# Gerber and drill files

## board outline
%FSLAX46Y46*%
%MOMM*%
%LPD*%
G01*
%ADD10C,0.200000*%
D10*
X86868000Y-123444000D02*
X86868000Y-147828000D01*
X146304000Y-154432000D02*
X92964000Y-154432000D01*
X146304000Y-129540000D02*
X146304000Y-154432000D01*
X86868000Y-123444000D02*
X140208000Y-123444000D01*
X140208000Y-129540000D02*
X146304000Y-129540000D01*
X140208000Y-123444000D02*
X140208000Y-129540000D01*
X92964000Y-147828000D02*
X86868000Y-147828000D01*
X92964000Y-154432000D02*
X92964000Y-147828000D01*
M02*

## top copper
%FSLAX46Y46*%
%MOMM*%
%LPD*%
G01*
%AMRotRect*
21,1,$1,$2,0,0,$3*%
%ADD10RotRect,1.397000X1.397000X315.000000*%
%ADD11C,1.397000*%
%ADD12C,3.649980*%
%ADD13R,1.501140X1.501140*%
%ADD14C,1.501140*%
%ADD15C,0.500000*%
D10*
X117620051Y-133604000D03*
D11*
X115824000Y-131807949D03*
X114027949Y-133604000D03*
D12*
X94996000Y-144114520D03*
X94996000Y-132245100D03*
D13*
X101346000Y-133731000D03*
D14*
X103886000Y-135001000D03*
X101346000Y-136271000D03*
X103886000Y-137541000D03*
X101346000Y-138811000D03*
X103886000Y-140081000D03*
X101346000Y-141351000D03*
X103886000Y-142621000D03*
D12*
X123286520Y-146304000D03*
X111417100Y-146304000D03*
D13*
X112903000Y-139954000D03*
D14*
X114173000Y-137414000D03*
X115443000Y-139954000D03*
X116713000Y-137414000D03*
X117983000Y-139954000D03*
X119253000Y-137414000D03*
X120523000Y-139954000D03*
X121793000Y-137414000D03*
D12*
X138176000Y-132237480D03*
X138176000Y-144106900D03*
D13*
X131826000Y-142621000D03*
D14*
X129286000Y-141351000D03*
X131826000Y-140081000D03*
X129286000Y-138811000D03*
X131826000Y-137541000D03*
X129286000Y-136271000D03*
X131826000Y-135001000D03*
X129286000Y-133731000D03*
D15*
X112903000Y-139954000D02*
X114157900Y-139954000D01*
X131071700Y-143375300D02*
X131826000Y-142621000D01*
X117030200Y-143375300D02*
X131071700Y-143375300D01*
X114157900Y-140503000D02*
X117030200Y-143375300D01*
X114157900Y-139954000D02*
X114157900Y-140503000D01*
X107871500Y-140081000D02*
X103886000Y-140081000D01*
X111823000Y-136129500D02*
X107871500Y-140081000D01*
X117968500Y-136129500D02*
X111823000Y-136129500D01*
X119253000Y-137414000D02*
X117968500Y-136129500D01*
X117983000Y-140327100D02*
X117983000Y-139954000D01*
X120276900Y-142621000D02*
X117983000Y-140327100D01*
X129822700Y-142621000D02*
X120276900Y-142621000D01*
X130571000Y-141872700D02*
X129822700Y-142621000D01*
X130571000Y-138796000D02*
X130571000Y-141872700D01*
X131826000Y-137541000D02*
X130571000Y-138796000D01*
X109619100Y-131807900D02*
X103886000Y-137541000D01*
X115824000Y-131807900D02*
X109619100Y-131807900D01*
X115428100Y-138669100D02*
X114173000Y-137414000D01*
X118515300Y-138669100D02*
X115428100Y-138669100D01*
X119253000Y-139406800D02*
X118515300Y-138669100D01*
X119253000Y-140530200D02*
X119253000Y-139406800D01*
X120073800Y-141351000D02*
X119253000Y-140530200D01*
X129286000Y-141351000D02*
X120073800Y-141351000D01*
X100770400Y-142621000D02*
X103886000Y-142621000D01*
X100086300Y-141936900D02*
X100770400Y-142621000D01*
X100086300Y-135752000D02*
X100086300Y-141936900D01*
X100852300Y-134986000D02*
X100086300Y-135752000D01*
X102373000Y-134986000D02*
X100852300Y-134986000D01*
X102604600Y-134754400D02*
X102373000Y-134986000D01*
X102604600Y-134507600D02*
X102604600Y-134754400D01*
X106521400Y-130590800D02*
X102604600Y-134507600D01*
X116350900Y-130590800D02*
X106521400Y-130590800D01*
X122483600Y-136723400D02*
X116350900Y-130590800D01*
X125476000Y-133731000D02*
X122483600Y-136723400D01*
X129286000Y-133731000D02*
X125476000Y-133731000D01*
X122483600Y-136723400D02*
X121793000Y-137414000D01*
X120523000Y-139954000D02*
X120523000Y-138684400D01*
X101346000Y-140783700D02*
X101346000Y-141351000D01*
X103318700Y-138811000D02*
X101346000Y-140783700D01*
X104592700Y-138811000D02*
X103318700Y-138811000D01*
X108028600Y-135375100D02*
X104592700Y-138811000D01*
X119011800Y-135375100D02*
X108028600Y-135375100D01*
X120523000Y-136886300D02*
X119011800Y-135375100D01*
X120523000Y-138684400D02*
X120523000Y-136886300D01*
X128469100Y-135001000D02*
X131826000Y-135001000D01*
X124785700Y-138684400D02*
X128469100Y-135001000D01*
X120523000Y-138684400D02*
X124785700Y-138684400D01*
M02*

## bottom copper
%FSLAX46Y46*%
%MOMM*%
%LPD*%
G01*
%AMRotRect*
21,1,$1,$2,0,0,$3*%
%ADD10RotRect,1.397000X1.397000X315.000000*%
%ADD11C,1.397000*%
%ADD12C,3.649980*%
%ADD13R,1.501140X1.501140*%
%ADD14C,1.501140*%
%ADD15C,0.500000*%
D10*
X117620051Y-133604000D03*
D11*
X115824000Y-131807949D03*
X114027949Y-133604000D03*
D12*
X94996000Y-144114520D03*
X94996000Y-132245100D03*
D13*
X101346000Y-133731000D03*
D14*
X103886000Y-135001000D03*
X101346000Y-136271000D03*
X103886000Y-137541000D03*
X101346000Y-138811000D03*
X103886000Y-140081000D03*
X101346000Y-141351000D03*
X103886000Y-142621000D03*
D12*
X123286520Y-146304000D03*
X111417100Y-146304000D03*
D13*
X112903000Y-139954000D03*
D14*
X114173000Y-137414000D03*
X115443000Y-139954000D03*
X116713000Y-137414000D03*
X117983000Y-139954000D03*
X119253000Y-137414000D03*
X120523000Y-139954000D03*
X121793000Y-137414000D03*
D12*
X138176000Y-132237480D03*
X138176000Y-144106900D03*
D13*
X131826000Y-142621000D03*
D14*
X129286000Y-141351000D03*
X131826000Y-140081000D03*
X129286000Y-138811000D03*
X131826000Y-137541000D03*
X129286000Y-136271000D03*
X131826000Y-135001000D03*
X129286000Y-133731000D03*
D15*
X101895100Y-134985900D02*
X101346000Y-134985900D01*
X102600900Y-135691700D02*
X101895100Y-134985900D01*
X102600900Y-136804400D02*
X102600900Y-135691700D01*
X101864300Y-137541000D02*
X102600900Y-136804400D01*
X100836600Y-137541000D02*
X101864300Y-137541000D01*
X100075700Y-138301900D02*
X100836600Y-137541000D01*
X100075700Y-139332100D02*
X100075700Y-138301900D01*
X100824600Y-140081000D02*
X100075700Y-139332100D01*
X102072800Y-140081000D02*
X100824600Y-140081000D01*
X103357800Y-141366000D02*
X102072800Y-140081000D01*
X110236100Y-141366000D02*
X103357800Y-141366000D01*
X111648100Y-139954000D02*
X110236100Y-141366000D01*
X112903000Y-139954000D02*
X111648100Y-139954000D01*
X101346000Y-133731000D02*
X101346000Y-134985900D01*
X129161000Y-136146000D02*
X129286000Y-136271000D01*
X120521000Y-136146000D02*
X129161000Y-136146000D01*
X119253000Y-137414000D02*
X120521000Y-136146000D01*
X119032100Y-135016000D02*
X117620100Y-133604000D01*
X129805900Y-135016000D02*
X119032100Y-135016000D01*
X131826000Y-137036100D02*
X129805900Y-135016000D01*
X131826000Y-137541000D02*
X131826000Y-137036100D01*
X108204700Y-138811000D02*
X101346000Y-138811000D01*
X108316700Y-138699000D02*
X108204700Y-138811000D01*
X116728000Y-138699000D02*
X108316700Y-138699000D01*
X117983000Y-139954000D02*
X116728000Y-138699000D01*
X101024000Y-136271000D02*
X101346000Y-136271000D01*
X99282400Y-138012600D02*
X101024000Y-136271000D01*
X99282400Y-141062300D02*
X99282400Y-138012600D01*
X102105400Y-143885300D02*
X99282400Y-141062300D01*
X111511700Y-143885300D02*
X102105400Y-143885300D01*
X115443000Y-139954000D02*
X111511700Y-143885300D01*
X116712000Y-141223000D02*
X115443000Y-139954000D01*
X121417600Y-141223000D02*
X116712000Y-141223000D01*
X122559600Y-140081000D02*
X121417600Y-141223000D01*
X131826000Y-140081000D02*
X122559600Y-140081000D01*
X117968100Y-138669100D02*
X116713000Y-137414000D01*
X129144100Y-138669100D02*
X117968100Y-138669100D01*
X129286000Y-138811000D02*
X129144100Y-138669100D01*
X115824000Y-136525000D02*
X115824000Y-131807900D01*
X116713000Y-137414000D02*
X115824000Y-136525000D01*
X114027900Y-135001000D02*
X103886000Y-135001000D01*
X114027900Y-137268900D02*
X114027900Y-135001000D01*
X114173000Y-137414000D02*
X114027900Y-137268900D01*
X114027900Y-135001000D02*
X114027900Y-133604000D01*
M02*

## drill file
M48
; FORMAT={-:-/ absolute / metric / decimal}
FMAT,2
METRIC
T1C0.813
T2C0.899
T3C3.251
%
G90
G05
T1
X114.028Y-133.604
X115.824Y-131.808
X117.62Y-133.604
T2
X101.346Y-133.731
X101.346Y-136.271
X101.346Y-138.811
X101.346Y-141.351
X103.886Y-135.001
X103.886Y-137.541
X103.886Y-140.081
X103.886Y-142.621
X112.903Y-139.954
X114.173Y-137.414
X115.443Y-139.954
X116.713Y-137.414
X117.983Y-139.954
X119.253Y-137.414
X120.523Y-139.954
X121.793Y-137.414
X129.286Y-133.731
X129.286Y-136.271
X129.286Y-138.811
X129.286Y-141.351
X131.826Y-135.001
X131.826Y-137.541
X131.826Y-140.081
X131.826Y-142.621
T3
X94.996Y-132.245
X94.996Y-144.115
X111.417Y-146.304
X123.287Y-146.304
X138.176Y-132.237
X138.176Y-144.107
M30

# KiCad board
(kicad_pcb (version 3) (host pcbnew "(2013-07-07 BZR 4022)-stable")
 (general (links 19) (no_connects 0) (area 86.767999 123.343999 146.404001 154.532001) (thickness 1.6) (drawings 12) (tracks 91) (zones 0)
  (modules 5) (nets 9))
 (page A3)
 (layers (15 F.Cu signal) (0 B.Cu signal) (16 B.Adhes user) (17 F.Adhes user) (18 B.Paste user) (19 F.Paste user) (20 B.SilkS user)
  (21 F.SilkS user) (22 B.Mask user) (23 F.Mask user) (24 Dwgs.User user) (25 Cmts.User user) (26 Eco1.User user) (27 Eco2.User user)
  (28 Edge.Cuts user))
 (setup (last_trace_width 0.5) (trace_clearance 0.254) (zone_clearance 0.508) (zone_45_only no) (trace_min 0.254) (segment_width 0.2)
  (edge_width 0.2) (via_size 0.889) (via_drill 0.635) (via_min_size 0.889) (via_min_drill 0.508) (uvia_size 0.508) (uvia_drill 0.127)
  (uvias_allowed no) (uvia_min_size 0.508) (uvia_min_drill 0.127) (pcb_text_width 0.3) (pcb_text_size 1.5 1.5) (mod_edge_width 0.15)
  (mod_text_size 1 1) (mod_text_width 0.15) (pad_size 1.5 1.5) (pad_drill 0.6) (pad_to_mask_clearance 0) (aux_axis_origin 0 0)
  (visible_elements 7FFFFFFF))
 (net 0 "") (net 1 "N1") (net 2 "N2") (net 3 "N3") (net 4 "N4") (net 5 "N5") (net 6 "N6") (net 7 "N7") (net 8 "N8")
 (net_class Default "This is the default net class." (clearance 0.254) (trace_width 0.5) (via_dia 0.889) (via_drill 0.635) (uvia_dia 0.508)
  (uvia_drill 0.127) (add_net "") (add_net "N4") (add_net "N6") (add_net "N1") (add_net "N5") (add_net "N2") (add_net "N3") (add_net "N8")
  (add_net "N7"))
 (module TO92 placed (layer F.Cu) (at 115.824 133.604 315)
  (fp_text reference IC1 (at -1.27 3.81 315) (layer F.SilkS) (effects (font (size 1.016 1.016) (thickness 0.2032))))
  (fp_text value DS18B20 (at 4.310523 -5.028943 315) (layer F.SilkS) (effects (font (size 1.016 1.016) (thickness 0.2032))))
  (pad 1 thru_hole rect (at 1.27 -1.27 315) (size 1.397 1.397) (drill 0.8128) (layers *.Cu *.Mask F.SilkS) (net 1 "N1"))
  (pad 2 thru_hole circle (at -1.27 -1.27 315) (size 1.397 1.397) (drill 0.8128) (layers *.Cu *.Mask F.SilkS) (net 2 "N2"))
  (pad 3 thru_hole circle (at -1.27 1.27 315) (size 1.397 1.397) (drill 0.8128) (layers *.Cu *.Mask F.SilkS) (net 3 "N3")))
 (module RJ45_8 (layer F.Cu) (at 94.996 138.176 270)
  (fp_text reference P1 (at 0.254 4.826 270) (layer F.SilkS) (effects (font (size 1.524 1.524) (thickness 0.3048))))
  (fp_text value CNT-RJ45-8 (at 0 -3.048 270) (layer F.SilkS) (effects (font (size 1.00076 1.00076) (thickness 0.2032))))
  (pad Hole np_thru_hole circle (at 5.93852 0 270) (size 3.64998 3.64998) (drill 3.2512) (layers *.Cu *.SilkS *.Mask))
  (pad Hole np_thru_hole circle (at -5.9309 0 270) (size 3.64998 3.64998) (drill 3.2512) (layers *.Cu *.SilkS *.Mask))
  (pad 1 thru_hole rect (at -4.445 -6.35 270) (size 1.50114 1.50114) (drill 0.89916) (layers *.Cu *.Mask F.SilkS) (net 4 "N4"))
  (pad 2 thru_hole circle (at -3.175 -8.89 270) (size 1.50114 1.50114) (drill 0.89916) (layers *.Cu *.Mask F.SilkS) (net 3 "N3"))
  (pad 3 thru_hole circle (at -1.905 -6.35 270) (size 1.50114 1.50114) (drill 0.89916) (layers *.Cu *.Mask F.SilkS) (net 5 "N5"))
  (pad 4 thru_hole circle (at -0.635 -8.89 270) (size 1.50114 1.50114) (drill 0.89916) (layers *.Cu *.Mask F.SilkS) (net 2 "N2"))
  (pad 5 thru_hole circle (at 0.635 -6.35 270) (size 1.50114 1.50114) (drill 0.89916) (layers *.Cu *.Mask F.SilkS) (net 1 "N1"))
  (pad 6 thru_hole circle (at 1.905 -8.89 270) (size 1.50114 1.50114) (drill 0.89916) (layers *.Cu *.Mask F.SilkS) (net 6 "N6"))
  (pad 7 thru_hole circle (at 3.175 -6.35 270) (size 1.50114 1.50114) (drill 0.89916) (layers *.Cu *.Mask F.SilkS) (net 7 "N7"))
  (pad 8 thru_hole circle (at 4.445 -8.89 270) (size 1.50114 1.50114) (drill 0.89916) (layers *.Cu *.Mask F.SilkS) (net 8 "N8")))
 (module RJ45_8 (layer F.Cu) (at 117.348 146.304)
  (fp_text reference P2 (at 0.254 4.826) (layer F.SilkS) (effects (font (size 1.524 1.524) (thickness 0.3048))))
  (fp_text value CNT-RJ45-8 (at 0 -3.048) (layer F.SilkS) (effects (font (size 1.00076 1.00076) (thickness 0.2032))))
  (pad Hole np_thru_hole circle (at 5.93852 0) (size 3.64998 3.64998) (drill 3.2512) (layers *.Cu *.SilkS *.Mask))
  (pad Hole np_thru_hole circle (at -5.9309 0) (size 3.64998 3.64998) (drill 3.2512) (layers *.Cu *.SilkS *.Mask))
  (pad 1 thru_hole rect (at -4.445 -6.35) (size 1.50114 1.50114) (drill 0.89916) (layers *.Cu *.Mask F.SilkS) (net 4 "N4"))
  (pad 2 thru_hole circle (at -3.175 -8.89) (size 1.50114 1.50114) (drill 0.89916) (layers *.Cu *.Mask F.SilkS) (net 3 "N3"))
  (pad 3 thru_hole circle (at -1.905 -6.35) (size 1.50114 1.50114) (drill 0.89916) (layers *.Cu *.Mask F.SilkS) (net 5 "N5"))
  (pad 4 thru_hole circle (at -0.635 -8.89) (size 1.50114 1.50114) (drill 0.89916) (layers *.Cu *.Mask F.SilkS) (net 2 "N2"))
  (pad 5 thru_hole circle (at 0.635 -6.35) (size 1.50114 1.50114) (drill 0.89916) (layers *.Cu *.Mask F.SilkS) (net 1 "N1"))
  (pad 6 thru_hole circle (at 1.905 -8.89) (size 1.50114 1.50114) (drill 0.89916) (layers *.Cu *.Mask F.SilkS) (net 6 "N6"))
  (pad 7 thru_hole circle (at 3.175 -6.35) (size 1.50114 1.50114) (drill 0.89916) (layers *.Cu *.Mask F.SilkS) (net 7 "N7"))
  (pad 8 thru_hole circle (at 4.445 -8.89) (size 1.50114 1.50114) (drill 0.89916) (layers *.Cu *.Mask F.SilkS) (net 8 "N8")))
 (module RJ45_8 (layer F.Cu) (at 138.176 138.176 90)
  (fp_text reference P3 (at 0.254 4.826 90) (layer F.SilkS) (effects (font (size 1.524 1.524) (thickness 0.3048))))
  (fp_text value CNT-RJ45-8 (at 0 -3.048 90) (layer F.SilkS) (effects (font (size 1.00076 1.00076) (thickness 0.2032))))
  (pad Hole np_thru_hole circle (at 5.93852 0 90) (size 3.64998 3.64998) (drill 3.2512) (layers *.Cu *.SilkS *.Mask))
  (pad Hole np_thru_hole circle (at -5.9309 0 90) (size 3.64998 3.64998) (drill 3.2512) (layers *.Cu *.SilkS *.Mask))
  (pad 1 thru_hole rect (at -4.445 -6.35 90) (size 1.50114 1.50114) (drill 0.89916) (layers *.Cu *.Mask F.SilkS) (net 4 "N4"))
  (pad 2 thru_hole circle (at -3.175 -8.89 90) (size 1.50114 1.50114) (drill 0.89916) (layers *.Cu *.Mask F.SilkS) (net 3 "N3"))
  (pad 3 thru_hole circle (at -1.905 -6.35 90) (size 1.50114 1.50114) (drill 0.89916) (layers *.Cu *.Mask F.SilkS) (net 5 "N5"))
  (pad 4 thru_hole circle (at -0.635 -8.89 90) (size 1.50114 1.50114) (drill 0.89916) (layers *.Cu *.Mask F.SilkS) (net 2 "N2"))
  (pad 5 thru_hole circle (at 0.635 -6.35 90) (size 1.50114 1.50114) (drill 0.89916) (layers *.Cu *.Mask F.SilkS) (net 1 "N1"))
  (pad 6 thru_hole circle (at 1.905 -8.89 90) (size 1.50114 1.50114) (drill 0.89916) (layers *.Cu *.Mask F.SilkS) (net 6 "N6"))
  (pad 7 thru_hole circle (at 3.175 -6.35 90) (size 1.50114 1.50114) (drill 0.89916) (layers *.Cu *.Mask F.SilkS) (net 7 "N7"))
  (pad 8 thru_hole circle (at 4.445 -8.89 90) (size 1.50114 1.50114) (drill 0.89916) (layers *.Cu *.Mask F.SilkS) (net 8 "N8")))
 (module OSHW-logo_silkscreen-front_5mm (layer F.Cu) (at 128.524 148.844)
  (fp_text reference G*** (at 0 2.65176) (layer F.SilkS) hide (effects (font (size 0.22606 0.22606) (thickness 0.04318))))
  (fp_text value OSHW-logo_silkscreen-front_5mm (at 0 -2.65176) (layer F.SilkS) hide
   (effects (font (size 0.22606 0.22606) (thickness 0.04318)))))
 (gr_line (start 86.868 123.444) (end 86.868 147.828) (angle 90) (layer Edge.Cuts) (width 0.2))
 (gr_line (start 146.304 154.432) (end 92.964 154.432) (angle 90) (layer Edge.Cuts) (width 0.2))
 (gr_line (start 146.304 129.54) (end 146.304 154.432) (angle 90) (layer Edge.Cuts) (width 0.2))
 (gr_line (start 86.868 123.444) (end 140.208 123.444) (angle 90) (layer Edge.Cuts) (width 0.2))
 (gr_line (start 140.208 129.54) (end 146.304 129.54) (angle 90) (layer Edge.Cuts) (width 0.2))
 (gr_line (start 140.208 123.444) (end 140.208 129.54) (angle 90) (layer Edge.Cuts) (width 0.2))
 (gr_line (start 92.964 147.828) (end 86.868 147.828) (angle 90) (layer Edge.Cuts) (width 0.2))
 (gr_line (start 92.964 154.432) (end 92.964 147.828) (angle 90) (layer Edge.Cuts) (width 0.2))
 (segment (start 101.8951 134.9859) (end 101.346 134.9859) (width 0.5) (layer B.Cu) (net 4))
 (segment (start 102.6009 135.6917) (end 101.8951 134.9859) (width 0.5) (layer B.Cu) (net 4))
 (segment (start 102.6009 136.8044) (end 102.6009 135.6917) (width 0.5) (layer B.Cu) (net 4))
 (segment (start 101.8643 137.541) (end 102.6009 136.8044) (width 0.5) (layer B.Cu) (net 4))
 (segment (start 100.8366 137.541) (end 101.8643 137.541) (width 0.5) (layer B.Cu) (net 4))
 (segment (start 100.0757 138.3019) (end 100.8366 137.541) (width 0.5) (layer B.Cu) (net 4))
 (segment (start 100.0757 139.3321) (end 100.0757 138.3019) (width 0.5) (layer B.Cu) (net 4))
 (segment (start 100.8246 140.081) (end 100.0757 139.3321) (width 0.5) (layer B.Cu) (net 4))
 (segment (start 102.0728 140.081) (end 100.8246 140.081) (width 0.5) (layer B.Cu) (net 4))
 (segment (start 103.3578 141.366) (end 102.0728 140.081) (width 0.5) (layer B.Cu) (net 4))
 (segment (start 110.2361 141.366) (end 103.3578 141.366) (width 0.5) (layer B.Cu) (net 4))
 (segment (start 111.6481 139.954) (end 110.2361 141.366) (width 0.5) (layer B.Cu) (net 4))
 (segment (start 112.903 139.954) (end 111.6481 139.954) (width 0.5) (layer B.Cu) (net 4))
 (segment (start 101.346 133.731) (end 101.346 134.9859) (width 0.5) (layer B.Cu) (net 4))
 (segment (start 112.903 139.954) (end 114.1579 139.954) (width 0.5) (layer F.Cu) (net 4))
 (segment (start 131.0717 143.3753) (end 131.826 142.621) (width 0.5) (layer F.Cu) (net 4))
 (segment (start 117.0302 143.3753) (end 131.0717 143.3753) (width 0.5) (layer F.Cu) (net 4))
 (segment (start 114.1579 140.503) (end 117.0302 143.3753) (width 0.5) (layer F.Cu) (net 4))
 (segment (start 114.1579 139.954) (end 114.1579 140.503) (width 0.5) (layer F.Cu) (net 4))
 (segment (start 129.161 136.146) (end 129.286 136.271) (width 0.5) (layer B.Cu) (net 6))
 (segment (start 120.521 136.146) (end 129.161 136.146) (width 0.5) (layer B.Cu) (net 6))
 (segment (start 119.253 137.414) (end 120.521 136.146) (width 0.5) (layer B.Cu) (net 6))
 (segment (start 107.8715 140.081) (end 103.886 140.081) (width 0.5) (layer F.Cu) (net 6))
 (segment (start 111.823 136.1295) (end 107.8715 140.081) (width 0.5) (layer F.Cu) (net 6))
 (segment (start 117.9685 136.1295) (end 111.823 136.1295) (width 0.5) (layer F.Cu) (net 6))
 (segment (start 119.253 137.414) (end 117.9685 136.1295) (width 0.5) (layer F.Cu) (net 6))
 (segment (start 119.0321 135.016) (end 117.6201 133.604) (width 0.5) (layer B.Cu) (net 1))
 (segment (start 129.8059 135.016) (end 119.0321 135.016) (width 0.5) (layer B.Cu) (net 1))
 (segment (start 131.826 137.0361) (end 129.8059 135.016) (width 0.5) (layer B.Cu) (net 1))
 (segment (start 131.826 137.541) (end 131.826 137.0361) (width 0.5) (layer B.Cu) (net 1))
 (segment (start 117.983 140.3271) (end 117.983 139.954) (width 0.5) (layer F.Cu) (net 1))
 (segment (start 120.2769 142.621) (end 117.983 140.3271) (width 0.5) (layer F.Cu) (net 1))
 (segment (start 129.8227 142.621) (end 120.2769 142.621) (width 0.5) (layer F.Cu) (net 1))
 (segment (start 130.571 141.8727) (end 129.8227 142.621) (width 0.5) (layer F.Cu) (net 1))
 (segment (start 130.571 138.796) (end 130.571 141.8727) (width 0.5) (layer F.Cu) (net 1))
 (segment (start 131.826 137.541) (end 130.571 138.796) (width 0.5) (layer F.Cu) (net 1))
 (segment (start 108.2047 138.811) (end 101.346 138.811) (width 0.5) (layer B.Cu) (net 1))
 (segment (start 108.3167 138.699) (end 108.2047 138.811) (width 0.5) (layer B.Cu) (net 1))
 (segment (start 116.728 138.699) (end 108.3167 138.699) (width 0.5) (layer B.Cu) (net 1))
 (segment (start 117.983 139.954) (end 116.728 138.699) (width 0.5) (layer B.Cu) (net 1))
 (segment (start 101.024 136.271) (end 101.346 136.271) (width 0.5) (layer B.Cu) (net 5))
 (segment (start 99.2824 138.0126) (end 101.024 136.271) (width 0.5) (layer B.Cu) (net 5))
 (segment (start 99.2824 141.0623) (end 99.2824 138.0126) (width 0.5) (layer B.Cu) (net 5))
 (segment (start 102.1054 143.8853) (end 99.2824 141.0623) (width 0.5) (layer B.Cu) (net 5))
 (segment (start 111.5117 143.8853) (end 102.1054 143.8853) (width 0.5) (layer B.Cu) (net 5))
 (segment (start 115.443 139.954) (end 111.5117 143.8853) (width 0.5) (layer B.Cu) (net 5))
 (segment (start 116.712 141.223) (end 115.443 139.954) (width 0.5) (layer B.Cu) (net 5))
 (segment (start 121.4176 141.223) (end 116.712 141.223) (width 0.5) (layer B.Cu) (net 5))
 (segment (start 122.5596 140.081) (end 121.4176 141.223) (width 0.5) (layer B.Cu) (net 5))
 (segment (start 131.826 140.081) (end 122.5596 140.081) (width 0.5) (layer B.Cu) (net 5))
 (segment (start 117.9681 138.6691) (end 116.713 137.414) (width 0.5) (layer B.Cu) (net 2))
 (segment (start 129.1441 138.6691) (end 117.9681 138.6691) (width 0.5) (layer B.Cu) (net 2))
 (segment (start 129.286 138.811) (end 129.1441 138.6691) (width 0.5) (layer B.Cu) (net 2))
 (segment (start 115.824 136.525) (end 115.824 131.8079) (width 0.5) (layer B.Cu) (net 2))
 (segment (start 116.713 137.414) (end 115.824 136.525) (width 0.5) (layer B.Cu) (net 2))
 (segment (start 109.6191 131.8079) (end 103.886 137.541) (width 0.5) (layer F.Cu) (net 2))
 (segment (start 115.824 131.8079) (end 109.6191 131.8079) (width 0.5) (layer F.Cu) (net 2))
 (segment (start 114.0279 135.001) (end 103.886 135.001) (width 0.5) (layer B.Cu) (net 3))
 (segment (start 114.0279 137.2689) (end 114.0279 135.001) (width 0.5) (layer B.Cu) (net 3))
 (segment (start 114.173 137.414) (end 114.0279 137.2689) (width 0.5) (layer B.Cu) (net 3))
 (segment (start 114.0279 135.001) (end 114.0279 133.604) (width 0.5) (layer B.Cu) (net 3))
 (segment (start 115.4281 138.6691) (end 114.173 137.414) (width 0.5) (layer F.Cu) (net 3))
 (segment (start 118.5153 138.6691) (end 115.4281 138.6691) (width 0.5) (layer F.Cu) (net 3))
 (segment (start 119.253 139.4068) (end 118.5153 138.6691) (width 0.5) (layer F.Cu) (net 3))
 (segment (start 119.253 140.5302) (end 119.253 139.4068) (width 0.5) (layer F.Cu) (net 3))
 (segment (start 120.0738 141.351) (end 119.253 140.5302) (width 0.5) (layer F.Cu) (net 3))
 (segment (start 129.286 141.351) (end 120.0738 141.351) (width 0.5) (layer F.Cu) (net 3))
 (segment (start 100.7704 142.621) (end 103.886 142.621) (width 0.5) (layer F.Cu) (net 8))
 (segment (start 100.0863 141.9369) (end 100.7704 142.621) (width 0.5) (layer F.Cu) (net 8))
 (segment (start 100.0863 135.752) (end 100.0863 141.9369) (width 0.5) (layer F.Cu) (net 8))
 (segment (start 100.8523 134.986) (end 100.0863 135.752) (width 0.5) (layer F.Cu) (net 8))
 (segment (start 102.373 134.986) (end 100.8523 134.986) (width 0.5) (layer F.Cu) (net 8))
 (segment (start 102.6046 134.7544) (end 102.373 134.986) (width 0.5) (layer F.Cu) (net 8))
 (segment (start 102.6046 134.5076) (end 102.6046 134.7544) (width 0.5) (layer F.Cu) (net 8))
 (segment (start 106.5214 130.5908) (end 102.6046 134.5076) (width 0.5) (layer F.Cu) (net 8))
 (segment (start 116.3509 130.5908) (end 106.5214 130.5908) (width 0.5) (layer F.Cu) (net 8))
 (segment (start 122.4836 136.7234) (end 116.3509 130.5908) (width 0.5) (layer F.Cu) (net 8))
 (segment (start 125.476 133.731) (end 122.4836 136.7234) (width 0.5) (layer F.Cu) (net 8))
 (segment (start 129.286 133.731) (end 125.476 133.731) (width 0.5) (layer F.Cu) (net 8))
 (segment (start 122.4836 136.7234) (end 121.793 137.414) (width 0.5) (layer F.Cu) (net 8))
 (segment (start 120.523 139.954) (end 120.523 138.6844) (width 0.5) (layer F.Cu) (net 7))
 (segment (start 101.346 140.7837) (end 101.346 141.351) (width 0.5) (layer F.Cu) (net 7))
 (segment (start 103.3187 138.811) (end 101.346 140.7837) (width 0.5) (layer F.Cu) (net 7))
 (segment (start 104.5927 138.811) (end 103.3187 138.811) (width 0.5) (layer F.Cu) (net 7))
 (segment (start 108.0286 135.3751) (end 104.5927 138.811) (width 0.5) (layer F.Cu) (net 7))
 (segment (start 119.0118 135.3751) (end 108.0286 135.3751) (width 0.5) (layer F.Cu) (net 7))
 (segment (start 120.523 136.8863) (end 119.0118 135.3751) (width 0.5) (layer F.Cu) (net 7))
 (segment (start 120.523 138.6844) (end 120.523 136.8863) (width 0.5) (layer F.Cu) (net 7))
 (segment (start 128.4691 135.001) (end 131.826 135.001) (width 0.5) (layer F.Cu) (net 7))
 (segment (start 124.7857 138.6844) (end 128.4691 135.001) (width 0.5) (layer F.Cu) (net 7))
 (segment (start 120.523 138.6844) (end 124.7857 138.6844) (width 0.5) (layer F.Cu) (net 7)))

